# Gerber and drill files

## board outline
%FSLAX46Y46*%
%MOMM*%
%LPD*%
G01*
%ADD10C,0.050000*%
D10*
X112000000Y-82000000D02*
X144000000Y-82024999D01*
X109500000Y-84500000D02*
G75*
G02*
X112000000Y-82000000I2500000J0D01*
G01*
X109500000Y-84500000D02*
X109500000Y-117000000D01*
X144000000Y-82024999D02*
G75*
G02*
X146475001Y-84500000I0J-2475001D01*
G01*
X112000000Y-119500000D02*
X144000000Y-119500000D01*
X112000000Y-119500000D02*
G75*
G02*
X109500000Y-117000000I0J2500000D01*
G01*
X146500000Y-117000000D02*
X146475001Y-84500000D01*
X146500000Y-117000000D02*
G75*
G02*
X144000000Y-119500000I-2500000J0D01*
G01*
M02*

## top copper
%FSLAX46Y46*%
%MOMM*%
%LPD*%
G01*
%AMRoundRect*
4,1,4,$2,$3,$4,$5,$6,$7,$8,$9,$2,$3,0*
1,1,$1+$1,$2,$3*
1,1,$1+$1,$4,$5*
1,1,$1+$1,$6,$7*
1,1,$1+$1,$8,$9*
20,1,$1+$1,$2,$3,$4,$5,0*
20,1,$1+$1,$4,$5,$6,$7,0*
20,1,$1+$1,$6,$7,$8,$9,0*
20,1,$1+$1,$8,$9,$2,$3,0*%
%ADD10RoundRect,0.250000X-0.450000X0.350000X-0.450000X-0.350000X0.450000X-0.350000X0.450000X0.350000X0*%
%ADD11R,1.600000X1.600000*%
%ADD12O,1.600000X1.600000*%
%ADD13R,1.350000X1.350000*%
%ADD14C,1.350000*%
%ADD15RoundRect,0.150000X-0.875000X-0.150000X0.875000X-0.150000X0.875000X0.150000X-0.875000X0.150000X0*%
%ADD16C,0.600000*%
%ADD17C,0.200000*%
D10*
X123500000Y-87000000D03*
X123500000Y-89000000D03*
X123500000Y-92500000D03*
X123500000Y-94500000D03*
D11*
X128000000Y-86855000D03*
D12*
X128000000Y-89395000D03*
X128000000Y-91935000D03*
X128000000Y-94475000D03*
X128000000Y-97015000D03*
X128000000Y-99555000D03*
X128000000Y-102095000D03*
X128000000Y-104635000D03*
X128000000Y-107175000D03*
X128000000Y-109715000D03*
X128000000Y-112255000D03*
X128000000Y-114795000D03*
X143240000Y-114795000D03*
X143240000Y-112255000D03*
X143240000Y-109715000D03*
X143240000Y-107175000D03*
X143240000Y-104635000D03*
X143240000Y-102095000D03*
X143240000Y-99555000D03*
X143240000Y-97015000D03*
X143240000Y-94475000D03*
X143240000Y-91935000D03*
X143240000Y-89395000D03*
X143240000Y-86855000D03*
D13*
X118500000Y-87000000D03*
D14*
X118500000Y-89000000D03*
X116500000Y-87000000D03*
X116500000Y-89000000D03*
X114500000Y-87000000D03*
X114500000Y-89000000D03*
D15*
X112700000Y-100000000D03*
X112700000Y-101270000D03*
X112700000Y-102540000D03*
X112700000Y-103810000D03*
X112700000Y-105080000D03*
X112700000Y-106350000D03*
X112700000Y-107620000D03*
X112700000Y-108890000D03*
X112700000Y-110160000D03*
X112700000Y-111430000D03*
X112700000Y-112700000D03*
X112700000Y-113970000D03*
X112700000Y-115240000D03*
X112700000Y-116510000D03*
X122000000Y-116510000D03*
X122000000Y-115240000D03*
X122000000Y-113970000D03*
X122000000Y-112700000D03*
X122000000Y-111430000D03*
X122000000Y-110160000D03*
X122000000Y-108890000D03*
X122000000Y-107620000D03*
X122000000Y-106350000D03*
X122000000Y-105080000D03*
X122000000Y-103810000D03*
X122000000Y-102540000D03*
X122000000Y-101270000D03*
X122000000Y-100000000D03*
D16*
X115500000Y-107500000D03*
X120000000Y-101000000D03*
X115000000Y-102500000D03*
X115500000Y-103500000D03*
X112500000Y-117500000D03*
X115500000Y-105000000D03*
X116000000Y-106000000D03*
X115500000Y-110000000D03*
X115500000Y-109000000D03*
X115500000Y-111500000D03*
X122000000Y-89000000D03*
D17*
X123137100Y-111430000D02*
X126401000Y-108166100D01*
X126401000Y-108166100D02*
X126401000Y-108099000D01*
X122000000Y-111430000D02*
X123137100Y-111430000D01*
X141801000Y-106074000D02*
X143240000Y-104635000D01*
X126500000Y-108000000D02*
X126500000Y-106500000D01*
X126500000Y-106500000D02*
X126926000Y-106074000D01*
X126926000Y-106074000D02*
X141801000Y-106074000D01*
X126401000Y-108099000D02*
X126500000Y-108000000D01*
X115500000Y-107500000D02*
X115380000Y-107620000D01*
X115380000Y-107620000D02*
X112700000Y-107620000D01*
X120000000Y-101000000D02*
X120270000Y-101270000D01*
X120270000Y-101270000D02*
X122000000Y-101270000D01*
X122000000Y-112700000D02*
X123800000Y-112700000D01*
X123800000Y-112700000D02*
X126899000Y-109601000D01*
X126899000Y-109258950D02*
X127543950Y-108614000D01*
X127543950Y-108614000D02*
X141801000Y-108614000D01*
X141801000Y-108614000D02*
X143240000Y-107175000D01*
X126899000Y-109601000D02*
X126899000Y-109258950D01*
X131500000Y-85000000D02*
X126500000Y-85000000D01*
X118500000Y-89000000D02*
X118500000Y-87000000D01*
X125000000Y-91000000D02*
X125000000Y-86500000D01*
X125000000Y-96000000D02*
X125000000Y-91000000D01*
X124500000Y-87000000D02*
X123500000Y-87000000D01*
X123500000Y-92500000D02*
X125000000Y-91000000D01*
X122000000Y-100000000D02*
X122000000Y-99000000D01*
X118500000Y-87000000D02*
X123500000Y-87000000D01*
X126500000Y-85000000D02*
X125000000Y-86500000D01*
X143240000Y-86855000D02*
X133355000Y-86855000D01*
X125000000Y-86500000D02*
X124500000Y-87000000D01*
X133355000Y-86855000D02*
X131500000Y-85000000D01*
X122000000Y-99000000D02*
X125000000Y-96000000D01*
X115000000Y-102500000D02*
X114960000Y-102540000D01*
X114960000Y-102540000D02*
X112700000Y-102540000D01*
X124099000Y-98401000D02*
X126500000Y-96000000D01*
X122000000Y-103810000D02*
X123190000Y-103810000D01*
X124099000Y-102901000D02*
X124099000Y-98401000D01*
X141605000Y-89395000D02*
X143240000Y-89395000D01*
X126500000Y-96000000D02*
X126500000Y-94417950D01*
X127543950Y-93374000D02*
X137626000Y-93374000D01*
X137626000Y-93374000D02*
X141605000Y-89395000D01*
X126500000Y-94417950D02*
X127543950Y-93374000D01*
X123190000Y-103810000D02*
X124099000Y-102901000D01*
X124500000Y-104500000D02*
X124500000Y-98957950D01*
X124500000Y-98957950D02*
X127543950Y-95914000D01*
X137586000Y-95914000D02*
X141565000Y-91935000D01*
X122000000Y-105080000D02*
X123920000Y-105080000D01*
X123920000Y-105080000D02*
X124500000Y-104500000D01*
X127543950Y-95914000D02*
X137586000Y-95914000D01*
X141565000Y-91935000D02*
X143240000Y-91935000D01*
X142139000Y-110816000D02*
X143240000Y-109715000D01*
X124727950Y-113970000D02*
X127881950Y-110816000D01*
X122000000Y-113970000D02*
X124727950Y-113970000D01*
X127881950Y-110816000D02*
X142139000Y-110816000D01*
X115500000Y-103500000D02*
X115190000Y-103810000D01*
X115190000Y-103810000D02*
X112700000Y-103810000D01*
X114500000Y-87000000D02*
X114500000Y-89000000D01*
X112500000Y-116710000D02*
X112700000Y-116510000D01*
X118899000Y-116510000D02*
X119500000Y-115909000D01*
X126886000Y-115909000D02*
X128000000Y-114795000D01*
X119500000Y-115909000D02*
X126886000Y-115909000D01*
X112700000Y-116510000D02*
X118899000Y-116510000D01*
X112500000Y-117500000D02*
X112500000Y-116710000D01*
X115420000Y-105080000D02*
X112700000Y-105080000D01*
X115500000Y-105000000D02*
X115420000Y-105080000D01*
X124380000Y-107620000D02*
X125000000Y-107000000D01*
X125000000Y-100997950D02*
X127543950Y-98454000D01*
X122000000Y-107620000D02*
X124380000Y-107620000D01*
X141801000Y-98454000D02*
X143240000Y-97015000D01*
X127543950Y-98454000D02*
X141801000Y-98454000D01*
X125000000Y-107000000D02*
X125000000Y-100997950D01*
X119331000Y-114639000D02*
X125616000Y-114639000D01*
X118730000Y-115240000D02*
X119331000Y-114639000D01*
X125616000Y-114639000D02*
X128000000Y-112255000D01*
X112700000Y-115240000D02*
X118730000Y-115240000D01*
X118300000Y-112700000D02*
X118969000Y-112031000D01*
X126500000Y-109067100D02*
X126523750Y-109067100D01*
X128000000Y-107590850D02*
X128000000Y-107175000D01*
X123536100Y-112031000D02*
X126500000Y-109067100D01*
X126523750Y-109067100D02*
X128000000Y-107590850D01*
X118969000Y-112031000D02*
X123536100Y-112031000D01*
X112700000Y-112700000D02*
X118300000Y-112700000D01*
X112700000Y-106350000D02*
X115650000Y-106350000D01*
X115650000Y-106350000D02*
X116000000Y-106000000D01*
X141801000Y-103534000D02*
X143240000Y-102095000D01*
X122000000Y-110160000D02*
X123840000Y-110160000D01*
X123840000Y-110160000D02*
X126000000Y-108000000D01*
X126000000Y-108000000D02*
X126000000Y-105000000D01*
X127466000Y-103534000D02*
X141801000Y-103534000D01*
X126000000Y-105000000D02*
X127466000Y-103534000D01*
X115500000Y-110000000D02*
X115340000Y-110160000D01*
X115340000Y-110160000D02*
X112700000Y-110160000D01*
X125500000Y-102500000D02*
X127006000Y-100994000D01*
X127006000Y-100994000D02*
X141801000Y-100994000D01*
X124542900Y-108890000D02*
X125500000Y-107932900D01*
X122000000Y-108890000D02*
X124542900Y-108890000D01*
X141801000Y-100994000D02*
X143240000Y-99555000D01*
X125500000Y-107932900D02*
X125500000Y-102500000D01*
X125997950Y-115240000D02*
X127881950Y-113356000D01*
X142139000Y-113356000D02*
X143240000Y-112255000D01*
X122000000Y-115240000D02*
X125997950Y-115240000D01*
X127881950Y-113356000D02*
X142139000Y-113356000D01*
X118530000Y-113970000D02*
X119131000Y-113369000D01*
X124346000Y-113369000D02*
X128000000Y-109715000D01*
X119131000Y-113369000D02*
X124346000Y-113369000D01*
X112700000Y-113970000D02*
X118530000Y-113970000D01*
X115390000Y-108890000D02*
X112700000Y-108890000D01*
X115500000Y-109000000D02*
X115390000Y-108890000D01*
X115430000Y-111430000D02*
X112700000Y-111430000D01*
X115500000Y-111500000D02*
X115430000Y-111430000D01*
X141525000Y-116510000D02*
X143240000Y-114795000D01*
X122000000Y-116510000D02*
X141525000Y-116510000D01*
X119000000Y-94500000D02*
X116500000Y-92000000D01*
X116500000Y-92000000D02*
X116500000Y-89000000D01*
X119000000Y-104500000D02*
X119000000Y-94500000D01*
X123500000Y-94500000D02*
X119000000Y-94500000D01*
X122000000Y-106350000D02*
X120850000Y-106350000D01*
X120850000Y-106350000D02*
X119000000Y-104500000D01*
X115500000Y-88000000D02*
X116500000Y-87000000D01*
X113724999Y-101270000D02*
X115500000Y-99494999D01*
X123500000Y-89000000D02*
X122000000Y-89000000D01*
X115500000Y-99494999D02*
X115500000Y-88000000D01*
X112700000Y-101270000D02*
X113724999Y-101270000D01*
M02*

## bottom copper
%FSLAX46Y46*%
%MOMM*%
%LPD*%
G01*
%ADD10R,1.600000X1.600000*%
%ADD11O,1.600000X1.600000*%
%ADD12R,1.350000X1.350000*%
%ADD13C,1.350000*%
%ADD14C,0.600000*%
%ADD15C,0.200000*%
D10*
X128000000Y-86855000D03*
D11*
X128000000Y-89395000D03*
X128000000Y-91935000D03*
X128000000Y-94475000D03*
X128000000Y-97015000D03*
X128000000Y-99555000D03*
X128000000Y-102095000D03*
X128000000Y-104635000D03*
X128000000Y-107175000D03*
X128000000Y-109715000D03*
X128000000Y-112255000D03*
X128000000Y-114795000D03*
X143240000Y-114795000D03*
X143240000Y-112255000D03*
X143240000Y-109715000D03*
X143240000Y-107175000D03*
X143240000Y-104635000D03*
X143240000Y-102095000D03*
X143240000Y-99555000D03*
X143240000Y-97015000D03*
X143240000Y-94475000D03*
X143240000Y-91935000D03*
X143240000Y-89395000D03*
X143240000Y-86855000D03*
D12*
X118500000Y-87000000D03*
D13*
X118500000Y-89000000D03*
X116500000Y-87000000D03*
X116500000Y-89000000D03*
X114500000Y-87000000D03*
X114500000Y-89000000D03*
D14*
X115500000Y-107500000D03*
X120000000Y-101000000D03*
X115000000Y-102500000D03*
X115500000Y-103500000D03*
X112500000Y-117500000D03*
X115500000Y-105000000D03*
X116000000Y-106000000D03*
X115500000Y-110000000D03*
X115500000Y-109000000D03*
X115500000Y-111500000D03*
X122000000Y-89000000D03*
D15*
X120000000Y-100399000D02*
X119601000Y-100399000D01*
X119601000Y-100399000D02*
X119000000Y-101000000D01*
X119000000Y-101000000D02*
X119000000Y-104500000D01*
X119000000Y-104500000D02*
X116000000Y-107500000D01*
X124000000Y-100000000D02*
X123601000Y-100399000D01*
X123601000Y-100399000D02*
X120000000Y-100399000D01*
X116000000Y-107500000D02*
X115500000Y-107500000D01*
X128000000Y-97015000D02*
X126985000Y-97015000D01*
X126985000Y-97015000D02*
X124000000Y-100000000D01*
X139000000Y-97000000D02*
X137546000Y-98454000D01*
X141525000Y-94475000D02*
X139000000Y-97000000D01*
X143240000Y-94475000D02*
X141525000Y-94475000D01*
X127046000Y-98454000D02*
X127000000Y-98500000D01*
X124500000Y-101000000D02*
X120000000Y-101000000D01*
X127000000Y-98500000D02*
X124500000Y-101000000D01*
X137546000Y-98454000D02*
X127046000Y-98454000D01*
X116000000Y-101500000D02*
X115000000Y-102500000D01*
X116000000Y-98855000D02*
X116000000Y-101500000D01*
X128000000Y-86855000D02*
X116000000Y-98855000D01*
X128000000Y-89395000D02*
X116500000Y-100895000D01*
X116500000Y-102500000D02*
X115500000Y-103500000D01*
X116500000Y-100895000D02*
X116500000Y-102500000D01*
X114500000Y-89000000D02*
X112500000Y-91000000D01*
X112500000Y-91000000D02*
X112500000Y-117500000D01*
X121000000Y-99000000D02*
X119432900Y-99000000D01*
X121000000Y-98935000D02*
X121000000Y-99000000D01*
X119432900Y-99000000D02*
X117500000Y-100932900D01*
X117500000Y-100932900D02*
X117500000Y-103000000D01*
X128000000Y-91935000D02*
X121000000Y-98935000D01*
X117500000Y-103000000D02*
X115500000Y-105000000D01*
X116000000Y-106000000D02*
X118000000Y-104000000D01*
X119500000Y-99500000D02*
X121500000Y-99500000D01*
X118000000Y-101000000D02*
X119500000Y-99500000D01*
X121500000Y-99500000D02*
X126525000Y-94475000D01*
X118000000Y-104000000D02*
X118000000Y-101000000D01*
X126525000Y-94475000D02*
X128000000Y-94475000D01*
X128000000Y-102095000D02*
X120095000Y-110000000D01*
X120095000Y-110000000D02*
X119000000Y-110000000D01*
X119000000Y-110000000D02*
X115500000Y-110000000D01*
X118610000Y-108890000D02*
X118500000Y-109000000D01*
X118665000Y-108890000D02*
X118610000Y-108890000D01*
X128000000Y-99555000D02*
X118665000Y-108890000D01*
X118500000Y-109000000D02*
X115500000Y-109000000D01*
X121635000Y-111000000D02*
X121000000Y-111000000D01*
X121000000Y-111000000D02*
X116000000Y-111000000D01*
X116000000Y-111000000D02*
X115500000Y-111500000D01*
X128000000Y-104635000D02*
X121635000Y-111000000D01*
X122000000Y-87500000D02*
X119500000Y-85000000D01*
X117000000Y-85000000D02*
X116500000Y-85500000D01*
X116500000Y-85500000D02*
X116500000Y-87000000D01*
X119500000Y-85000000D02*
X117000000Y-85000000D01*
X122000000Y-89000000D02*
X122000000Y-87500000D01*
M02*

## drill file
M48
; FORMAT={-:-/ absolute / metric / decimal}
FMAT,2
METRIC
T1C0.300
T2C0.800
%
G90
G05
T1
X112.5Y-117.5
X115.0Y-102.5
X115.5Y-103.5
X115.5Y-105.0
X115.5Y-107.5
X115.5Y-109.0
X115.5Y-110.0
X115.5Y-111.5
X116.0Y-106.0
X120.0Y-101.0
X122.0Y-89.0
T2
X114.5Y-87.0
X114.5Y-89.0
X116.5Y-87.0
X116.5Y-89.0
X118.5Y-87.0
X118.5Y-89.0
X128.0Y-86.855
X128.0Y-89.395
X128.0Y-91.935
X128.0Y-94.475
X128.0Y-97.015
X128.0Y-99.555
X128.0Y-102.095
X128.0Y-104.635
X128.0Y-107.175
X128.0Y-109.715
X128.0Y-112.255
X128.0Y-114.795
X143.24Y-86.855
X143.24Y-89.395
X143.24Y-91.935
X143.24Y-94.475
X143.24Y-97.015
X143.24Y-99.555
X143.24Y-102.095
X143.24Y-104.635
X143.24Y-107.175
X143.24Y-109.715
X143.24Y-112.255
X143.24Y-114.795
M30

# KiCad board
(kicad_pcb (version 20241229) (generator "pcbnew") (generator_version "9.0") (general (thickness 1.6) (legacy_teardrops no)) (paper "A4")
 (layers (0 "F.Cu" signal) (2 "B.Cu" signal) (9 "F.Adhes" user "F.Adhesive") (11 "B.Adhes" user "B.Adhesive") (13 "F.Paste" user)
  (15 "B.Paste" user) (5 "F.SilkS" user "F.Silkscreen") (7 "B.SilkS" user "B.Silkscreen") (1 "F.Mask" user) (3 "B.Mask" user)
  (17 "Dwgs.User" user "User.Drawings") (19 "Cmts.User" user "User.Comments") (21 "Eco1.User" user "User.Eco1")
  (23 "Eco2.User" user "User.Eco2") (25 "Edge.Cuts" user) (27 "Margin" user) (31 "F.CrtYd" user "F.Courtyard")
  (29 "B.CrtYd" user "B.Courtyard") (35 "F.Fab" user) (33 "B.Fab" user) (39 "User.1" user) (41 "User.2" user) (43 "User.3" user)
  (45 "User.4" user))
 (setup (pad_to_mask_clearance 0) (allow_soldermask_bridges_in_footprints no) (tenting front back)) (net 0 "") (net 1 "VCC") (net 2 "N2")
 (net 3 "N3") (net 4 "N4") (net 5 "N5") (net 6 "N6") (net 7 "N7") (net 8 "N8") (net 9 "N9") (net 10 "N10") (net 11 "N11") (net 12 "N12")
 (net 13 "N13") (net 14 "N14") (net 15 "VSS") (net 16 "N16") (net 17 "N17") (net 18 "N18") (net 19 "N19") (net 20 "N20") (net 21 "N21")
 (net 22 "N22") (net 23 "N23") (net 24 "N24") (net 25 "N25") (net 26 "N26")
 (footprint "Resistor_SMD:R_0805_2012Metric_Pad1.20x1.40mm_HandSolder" (layer "F.Cu") (at 123.5 88 -90)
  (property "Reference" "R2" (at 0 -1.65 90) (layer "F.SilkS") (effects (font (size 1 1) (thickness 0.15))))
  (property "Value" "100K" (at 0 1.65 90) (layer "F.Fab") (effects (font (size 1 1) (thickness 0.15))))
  (pad "1" smd roundrect (at -1 0 270) (size 1.2 1.4) (layers "F.Cu" "F.Mask" "F.Paste") (roundrect_rratio 0.208333) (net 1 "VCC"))
  (pad "2" smd roundrect (at 1 0 270) (size 1.2 1.4) (layers "F.Cu" "F.Mask" "F.Paste") (roundrect_rratio 0.208333) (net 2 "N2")))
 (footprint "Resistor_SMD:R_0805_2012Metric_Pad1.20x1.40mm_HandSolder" (layer "F.Cu") (at 123.5 93.5 -90)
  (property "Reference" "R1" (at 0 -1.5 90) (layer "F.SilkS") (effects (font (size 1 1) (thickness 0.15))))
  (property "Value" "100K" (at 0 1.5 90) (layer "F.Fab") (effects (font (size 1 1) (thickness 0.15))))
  (pad "1" smd roundrect (at -1 0 270) (size 1.2 1.4) (layers "F.Cu" "F.Mask" "F.Paste") (roundrect_rratio 0.208333) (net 1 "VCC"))
  (pad "2" smd roundrect (at 1 0 270) (size 1.2 1.4) (layers "F.Cu" "F.Mask" "F.Paste") (roundrect_rratio 0.208333) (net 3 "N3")))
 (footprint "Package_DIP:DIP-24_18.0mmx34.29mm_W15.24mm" (layer "F.Cu") (at 128 86.855)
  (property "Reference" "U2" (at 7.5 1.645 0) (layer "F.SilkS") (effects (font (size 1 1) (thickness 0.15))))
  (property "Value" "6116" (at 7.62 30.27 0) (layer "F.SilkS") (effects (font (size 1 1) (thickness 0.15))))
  (pad "1" thru_hole rect (at 0 0) (size 1.6 1.6) (drill 0.8) (layers "*.Cu" "*.Mask") (remove_unused_layers no) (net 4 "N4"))
  (pad "2" thru_hole oval (at 0 2.54) (size 1.6 1.6) (drill 0.8) (layers "*.Cu" "*.Mask") (remove_unused_layers no) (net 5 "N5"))
  (pad "3" thru_hole oval (at 0 5.08) (size 1.6 1.6) (drill 0.8) (layers "*.Cu" "*.Mask") (remove_unused_layers no) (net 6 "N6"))
  (pad "4" thru_hole oval (at 0 7.62) (size 1.6 1.6) (drill 0.8) (layers "*.Cu" "*.Mask") (remove_unused_layers no) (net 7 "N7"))
  (pad "5" thru_hole oval (at 0 10.16) (size 1.6 1.6) (drill 0.8) (layers "*.Cu" "*.Mask") (remove_unused_layers no) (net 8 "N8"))
  (pad "6" thru_hole oval (at 0 12.7) (size 1.6 1.6) (drill 0.8) (layers "*.Cu" "*.Mask") (remove_unused_layers no) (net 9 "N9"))
  (pad "7" thru_hole oval (at 0 15.24) (size 1.6 1.6) (drill 0.8) (layers "*.Cu" "*.Mask") (remove_unused_layers no) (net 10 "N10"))
  (pad "8" thru_hole oval (at 0 17.78) (size 1.6 1.6) (drill 0.8) (layers "*.Cu" "*.Mask") (remove_unused_layers no) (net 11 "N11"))
  (pad "9" thru_hole oval (at 0 20.32) (size 1.6 1.6) (drill 0.8) (layers "*.Cu" "*.Mask") (remove_unused_layers no) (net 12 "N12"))
  (pad "10" thru_hole oval (at 0 22.86) (size 1.6 1.6) (drill 0.8) (layers "*.Cu" "*.Mask") (remove_unused_layers no) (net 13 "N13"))
  (pad "11" thru_hole oval (at 0 25.4) (size 1.6 1.6) (drill 0.8) (layers "*.Cu" "*.Mask") (remove_unused_layers no) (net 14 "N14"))
  (pad "12" thru_hole oval (at 0 27.94) (size 1.6 1.6) (drill 0.8) (layers "*.Cu" "*.Mask") (remove_unused_layers no) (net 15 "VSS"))
  (pad "13" thru_hole oval (at 15.24 27.94) (size 1.6 1.6) (drill 0.8) (layers "*.Cu" "*.Mask") (remove_unused_layers no) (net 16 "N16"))
  (pad "14" thru_hole oval (at 15.24 25.4) (size 1.6 1.6) (drill 0.8) (layers "*.Cu" "*.Mask") (remove_unused_layers no) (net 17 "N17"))
  (pad "15" thru_hole oval (at 15.24 22.86) (size 1.6 1.6) (drill 0.8) (layers "*.Cu" "*.Mask") (remove_unused_layers no) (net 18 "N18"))
  (pad "16" thru_hole oval (at 15.24 20.32) (size 1.6 1.6) (drill 0.8) (layers "*.Cu" "*.Mask") (remove_unused_layers no) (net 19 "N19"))
  (pad "17" thru_hole oval (at 15.24 17.78) (size 1.6 1.6) (drill 0.8) (layers "*.Cu" "*.Mask") (remove_unused_layers no) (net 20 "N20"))
  (pad "18" thru_hole oval (at 15.24 15.24) (size 1.6 1.6) (drill 0.8) (layers "*.Cu" "*.Mask") (remove_unused_layers no) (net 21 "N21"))
  (pad "19" thru_hole oval (at 15.24 12.7) (size 1.6 1.6) (drill 0.8) (layers "*.Cu" "*.Mask") (remove_unused_layers no) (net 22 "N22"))
  (pad "20" thru_hole oval (at 15.24 10.16) (size 1.6 1.6) (drill 0.8) (layers "*.Cu" "*.Mask") (remove_unused_layers no) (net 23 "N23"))
  (pad "21" thru_hole oval (at 15.24 7.62) (size 1.6 1.6) (drill 0.8) (layers "*.Cu" "*.Mask") (remove_unused_layers no) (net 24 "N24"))
  (pad "22" thru_hole oval (at 15.24 5.08) (size 1.6 1.6) (drill 0.8) (layers "*.Cu" "*.Mask") (remove_unused_layers no) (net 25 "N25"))
  (pad "23" thru_hole oval (at 15.24 2.54) (size 1.6 1.6) (drill 0.8) (layers "*.Cu" "*.Mask") (remove_unused_layers no) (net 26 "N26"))
  (pad "24" thru_hole oval (at 15.24 0) (size 1.6 1.6) (drill 0.8) (layers "*.Cu" "*.Mask") (remove_unused_layers no) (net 1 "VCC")))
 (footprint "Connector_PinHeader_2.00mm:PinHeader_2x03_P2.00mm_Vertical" (layer "F.Cu") (at 118.5 87 -90)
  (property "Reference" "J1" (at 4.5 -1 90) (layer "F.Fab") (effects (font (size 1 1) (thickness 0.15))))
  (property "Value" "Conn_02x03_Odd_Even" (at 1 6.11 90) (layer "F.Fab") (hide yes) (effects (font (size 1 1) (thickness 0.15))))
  (pad "1" thru_hole rect (at 0 0 270) (size 1.35 1.35) (drill 0.8) (layers "*.Cu" "*.Mask") (remove_unused_layers no) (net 1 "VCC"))
  (pad "2" thru_hole circle (at 2 0 270) (size 1.35 1.35) (drill 0.8) (layers "*.Cu" "*.Mask") (remove_unused_layers no) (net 1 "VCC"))
  (pad "3" thru_hole circle (at 0 2 270) (size 1.35 1.35) (drill 0.8) (layers "*.Cu" "*.Mask") (remove_unused_layers no) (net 2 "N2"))
  (pad "4" thru_hole circle (at 2 2 270) (size 1.35 1.35) (drill 0.8) (layers "*.Cu" "*.Mask") (remove_unused_layers no) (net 3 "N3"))
  (pad "5" thru_hole circle (at 0 4 270) (size 1.35 1.35) (drill 0.8) (layers "*.Cu" "*.Mask") (remove_unused_layers no) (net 15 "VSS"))
  (pad "6" thru_hole circle (at 2 4 270) (size 1.35 1.35) (drill 0.8) (layers "*.Cu" "*.Mask") (remove_unused_layers no) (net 15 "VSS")))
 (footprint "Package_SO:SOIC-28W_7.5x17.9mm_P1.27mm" (layer "F.Cu") (at 117.35 108.255)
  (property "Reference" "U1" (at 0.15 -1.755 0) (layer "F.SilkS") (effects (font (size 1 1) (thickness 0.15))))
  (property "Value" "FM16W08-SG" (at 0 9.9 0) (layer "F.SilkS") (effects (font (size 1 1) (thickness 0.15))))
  (pad "1" smd roundrect (at -4.65 -8.255) (size 2.05 0.6) (layers "F.Cu" "F.Mask" "F.Paste") (roundrect_rratio 0.25))
  (pad "2" smd roundrect (at -4.65 -6.985) (size 2.05 0.6) (layers "F.Cu" "F.Mask" "F.Paste") (roundrect_rratio 0.25) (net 2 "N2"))
  (pad "3" smd roundrect (at -4.65 -5.715) (size 2.05 0.6) (layers "F.Cu" "F.Mask" "F.Paste") (roundrect_rratio 0.25) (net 4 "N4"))
  (pad "4" smd roundrect (at -4.65 -4.445) (size 2.05 0.6) (layers "F.Cu" "F.Mask" "F.Paste") (roundrect_rratio 0.25) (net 5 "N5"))
  (pad "5" smd roundrect (at -4.65 -3.175) (size 2.05 0.6) (layers "F.Cu" "F.Mask" "F.Paste") (roundrect_rratio 0.25) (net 6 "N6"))
  (pad "6" smd roundrect (at -4.65 -1.905) (size 2.05 0.6) (layers "F.Cu" "F.Mask" "F.Paste") (roundrect_rratio 0.25) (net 7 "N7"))
  (pad "7" smd roundrect (at -4.65 -0.635) (size 2.05 0.6) (layers "F.Cu" "F.Mask" "F.Paste") (roundrect_rratio 0.25) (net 8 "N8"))
  (pad "8" smd roundrect (at -4.65 0.635) (size 2.05 0.6) (layers "F.Cu" "F.Mask" "F.Paste") (roundrect_rratio 0.25) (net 9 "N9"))
  (pad "9" smd roundrect (at -4.65 1.905) (size 2.05 0.6) (layers "F.Cu" "F.Mask" "F.Paste") (roundrect_rratio 0.25) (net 10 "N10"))
  (pad "10" smd roundrect (at -4.65 3.175) (size 2.05 0.6) (layers "F.Cu" "F.Mask" "F.Paste") (roundrect_rratio 0.25) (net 11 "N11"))
  (pad "11" smd roundrect (at -4.65 4.445) (size 2.05 0.6) (layers "F.Cu" "F.Mask" "F.Paste") (roundrect_rratio 0.25) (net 12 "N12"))
  (pad "12" smd roundrect (at -4.65 5.715) (size 2.05 0.6) (layers "F.Cu" "F.Mask" "F.Paste") (roundrect_rratio 0.25) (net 13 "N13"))
  (pad "13" smd roundrect (at -4.65 6.985) (size 2.05 0.6) (layers "F.Cu" "F.Mask" "F.Paste") (roundrect_rratio 0.25) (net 14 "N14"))
  (pad "14" smd roundrect (at -4.65 8.255) (size 2.05 0.6) (layers "F.Cu" "F.Mask" "F.Paste") (roundrect_rratio 0.25) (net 15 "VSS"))
  (pad "15" smd roundrect (at 4.65 8.255) (size 2.05 0.6) (layers "F.Cu" "F.Mask" "F.Paste") (roundrect_rratio 0.25) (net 16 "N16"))
  (pad "16" smd roundrect (at 4.65 6.985) (size 2.05 0.6) (layers "F.Cu" "F.Mask" "F.Paste") (roundrect_rratio 0.25) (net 17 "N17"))
  (pad "17" smd roundrect (at 4.65 5.715) (size 2.05 0.6) (layers "F.Cu" "F.Mask" "F.Paste") (roundrect_rratio 0.25) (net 18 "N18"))
  (pad "18" smd roundrect (at 4.65 4.445) (size 2.05 0.6) (layers "F.Cu" "F.Mask" "F.Paste") (roundrect_rratio 0.25) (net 19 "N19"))
  (pad "19" smd roundrect (at 4.65 3.175) (size 2.05 0.6) (layers "F.Cu" "F.Mask" "F.Paste") (roundrect_rratio 0.25) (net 20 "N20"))
  (pad "20" smd roundrect (at 4.65 1.905) (size 2.05 0.6) (layers "F.Cu" "F.Mask" "F.Paste") (roundrect_rratio 0.25) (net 21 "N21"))
  (pad "21" smd roundrect (at 4.65 0.635) (size 2.05 0.6) (layers "F.Cu" "F.Mask" "F.Paste") (roundrect_rratio 0.25) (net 22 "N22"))
  (pad "22" smd roundrect (at 4.65 -0.635) (size 2.05 0.6) (layers "F.Cu" "F.Mask" "F.Paste") (roundrect_rratio 0.25) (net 23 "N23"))
  (pad "23" smd roundrect (at 4.65 -1.905) (size 2.05 0.6) (layers "F.Cu" "F.Mask" "F.Paste") (roundrect_rratio 0.25) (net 3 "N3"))
  (pad "24" smd roundrect (at 4.65 -3.175) (size 2.05 0.6) (layers "F.Cu" "F.Mask" "F.Paste") (roundrect_rratio 0.25) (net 25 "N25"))
  (pad "25" smd roundrect (at 4.65 -4.445) (size 2.05 0.6) (layers "F.Cu" "F.Mask" "F.Paste") (roundrect_rratio 0.25) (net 26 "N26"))
  (pad "26" smd roundrect (at 4.65 -5.715) (size 2.05 0.6) (layers "F.Cu" "F.Mask" "F.Paste") (roundrect_rratio 0.25))
  (pad "27" smd roundrect (at 4.65 -6.985) (size 2.05 0.6) (layers "F.Cu" "F.Mask" "F.Paste") (roundrect_rratio 0.25) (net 24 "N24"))
  (pad "28" smd roundrect (at 4.65 -8.255) (size 2.05 0.6) (layers "F.Cu" "F.Mask" "F.Paste") (roundrect_rratio 0.25) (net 1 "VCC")))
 (gr_line (start 112 82) (end 144 82.024999) (stroke (width 0.05) (type default)) (layer "Edge.Cuts"))
 (gr_arc (start 109.5 84.5) (mid 110.232233 82.732233) (end 112 82) (stroke (width 0.05) (type default)) (layer "Edge.Cuts"))
 (gr_line (start 109.5 84.5) (end 109.5 117) (stroke (width 0.05) (type default)) (layer "Edge.Cuts"))
 (gr_arc (start 144 82.024999) (mid 145.75009 82.74991) (end 146.475001 84.5) (stroke (width 0.05) (type solid)) (layer "Edge.Cuts"))
 (gr_line (start 112 119.5) (end 144 119.5) (stroke (width 0.05) (type default)) (layer "Edge.Cuts"))
 (gr_arc (start 112 119.5) (mid 110.232233 118.767767) (end 109.5 117) (stroke (width 0.05) (type solid)) (layer "Edge.Cuts"))
 (gr_line (start 146.5 117) (end 146.475001 84.5) (stroke (width 0.05) (type default)) (layer "Edge.Cuts"))
 (gr_arc (start 146.5 117) (mid 145.767767 118.767767) (end 144 119.5) (stroke (width 0.05) (type default)) (layer "Edge.Cuts"))
 (segment (start 123.1371 111.43) (end 126.401 108.1661) (width 0.2) (layer "F.Cu") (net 20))
 (segment (start 126.401 108.1661) (end 126.401 108.099) (width 0.2) (layer "F.Cu") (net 20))
 (segment (start 122 111.43) (end 123.1371 111.43) (width 0.2) (layer "F.Cu") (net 20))
 (segment (start 141.801 106.074) (end 143.24 104.635) (width 0.2) (layer "F.Cu") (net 20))
 (segment (start 126.5 108) (end 126.5 106.5) (width 0.2) (layer "F.Cu") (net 20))
 (segment (start 126.5 106.5) (end 126.926 106.074) (width 0.2) (layer "F.Cu") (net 20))
 (segment (start 126.926 106.074) (end 141.801 106.074) (width 0.2) (layer "F.Cu") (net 20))
 (segment (start 126.401 108.099) (end 126.5 108) (width 0.2) (layer "F.Cu") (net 20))
 (segment (start 115.5 107.5) (end 115.38 107.62) (width 0.2) (layer "F.Cu") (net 8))
 (segment (start 115.38 107.62) (end 112.7 107.62) (width 0.2) (layer "F.Cu") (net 8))
 (via (at 115.5 107.5) (size 0.6) (drill 0.3) (layers "F.Cu" "B.Cu") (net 8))
 (segment (start 120 100.399) (end 119.601 100.399) (width 0.2) (layer "B.Cu") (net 8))
 (segment (start 119.601 100.399) (end 119 101) (width 0.2) (layer "B.Cu") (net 8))
 (segment (start 119 101) (end 119 104.5) (width 0.2) (layer "B.Cu") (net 8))
 (segment (start 119 104.5) (end 116 107.5) (width 0.2) (layer "B.Cu") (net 8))
 (segment (start 124 100) (end 123.601 100.399) (width 0.2) (layer "B.Cu") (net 8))
 (segment (start 123.601 100.399) (end 120 100.399) (width 0.2) (layer "B.Cu") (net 8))
 (segment (start 116 107.5) (end 115.5 107.5) (width 0.2) (layer "B.Cu") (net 8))
 (segment (start 128 97.015) (end 126.985 97.015) (width 0.2) (layer "B.Cu") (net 8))
 (segment (start 126.985 97.015) (end 124 100) (width 0.2) (layer "B.Cu") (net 8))
 (segment (start 120 101) (end 120.27 101.27) (width 0.2) (layer "F.Cu") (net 24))
 (segment (start 120.27 101.27) (end 122 101.27) (width 0.2) (layer "F.Cu") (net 24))
 (via (at 120 101) (size 0.6) (drill 0.3) (layers "F.Cu" "B.Cu") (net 24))
 (segment (start 139 97) (end 137.546 98.454) (width 0.2) (layer "B.Cu") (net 24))
 (segment (start 141.525 94.475) (end 139 97) (width 0.2) (layer "B.Cu") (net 24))
 (segment (start 143.24 94.475) (end 141.525 94.475) (width 0.2) (layer "B.Cu") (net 24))
 (segment (start 127.046 98.454) (end 127 98.5) (width 0.2) (layer "B.Cu") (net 24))
 (segment (start 124.5 101) (end 120 101) (width 0.2) (layer "B.Cu") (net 24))
 (segment (start 127 98.5) (end 124.5 101) (width 0.2) (layer "B.Cu") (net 24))
 (segment (start 137.546 98.454) (end 127.046 98.454) (width 0.2) (layer "B.Cu") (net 24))
 (segment (start 122 112.7) (end 123.8 112.7) (width 0.2) (layer "F.Cu") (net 19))
 (segment (start 123.8 112.7) (end 126.899 109.601) (width 0.2) (layer "F.Cu") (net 19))
 (segment (start 126.899 109.25895) (end 127.54395 108.614) (width 0.2) (layer "F.Cu") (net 19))
 (segment (start 127.54395 108.614) (end 141.801 108.614) (width 0.2) (layer "F.Cu") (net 19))
 (segment (start 141.801 108.614) (end 143.24 107.175) (width 0.2) (layer "F.Cu") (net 19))
 (segment (start 126.899 109.601) (end 126.899 109.25895) (width 0.2) (layer "F.Cu") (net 19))
 (segment (start 131.5 85) (end 126.5 85) (width 0.2) (layer "F.Cu") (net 1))
 (segment (start 118.5 89) (end 118.5 87) (width 0.2) (layer "F.Cu") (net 1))
 (segment (start 125 91) (end 125 86.5) (width 0.2) (layer "F.Cu") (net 1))
 (segment (start 125 96) (end 125 91) (width 0.2) (layer "F.Cu") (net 1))
 (segment (start 124.5 87) (end 123.5 87) (width 0.2) (layer "F.Cu") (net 1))
 (segment (start 123.5 92.5) (end 125 91) (width 0.2) (layer "F.Cu") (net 1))
 (segment (start 122 100) (end 122 99) (width 0.2) (layer "F.Cu") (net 1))
 (segment (start 118.5 87) (end 123.5 87) (width 0.2) (layer "F.Cu") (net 1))
 (segment (start 126.5 85) (end 125 86.5) (width 0.2) (layer "F.Cu") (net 1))
 (segment (start 143.24 86.855) (end 133.355 86.855) (width 0.2) (layer "F.Cu") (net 1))
 (segment (start 125 86.5) (end 124.5 87) (width 0.2) (layer "F.Cu") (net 1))
 (segment (start 133.355 86.855) (end 131.5 85) (width 0.2) (layer "F.Cu") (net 1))
 (segment (start 122 99) (end 125 96) (width 0.2) (layer "F.Cu") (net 1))
 (segment (start 115 102.5) (end 114.96 102.54) (width 0.2) (layer "F.Cu") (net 4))
 (segment (start 114.96 102.54) (end 112.7 102.54) (width 0.2) (layer "F.Cu") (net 4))
 (via (at 115 102.5) (size 0.6) (drill 0.3) (layers "F.Cu" "B.Cu") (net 4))
 (segment (start 116 101.5) (end 115 102.5) (width 0.2) (layer "B.Cu") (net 4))
 (segment (start 116 98.855) (end 116 101.5) (width 0.2) (layer "B.Cu") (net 4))
 (segment (start 128 86.855) (end 116 98.855) (width 0.2) (layer "B.Cu") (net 4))
 (segment (start 124.099 98.401) (end 126.5 96) (width 0.2) (layer "F.Cu") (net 26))
 (segment (start 122 103.81) (end 123.19 103.81) (width 0.2) (layer "F.Cu") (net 26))
 (segment (start 124.099 102.901) (end 124.099 98.401) (width 0.2) (layer "F.Cu") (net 26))
 (segment (start 141.605 89.395) (end 143.24 89.395) (width 0.2) (layer "F.Cu") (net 26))
 (segment (start 126.5 96) (end 126.5 94.41795) (width 0.2) (layer "F.Cu") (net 26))
 (segment (start 127.54395 93.374) (end 137.626 93.374) (width 0.2) (layer "F.Cu") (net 26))
 (segment (start 137.626 93.374) (end 141.605 89.395) (width 0.2) (layer "F.Cu") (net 26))
 (segment (start 126.5 94.41795) (end 127.54395 93.374) (width 0.2) (layer "F.Cu") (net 26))
 (segment (start 123.19 103.81) (end 124.099 102.901) (width 0.2) (layer "F.Cu") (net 26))
 (segment (start 124.5 104.5) (end 124.5 98.95795) (width 0.2) (layer "F.Cu") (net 25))
 (segment (start 124.5 98.95795) (end 127.54395 95.914) (width 0.2) (layer "F.Cu") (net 25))
 (segment (start 137.586 95.914) (end 141.565 91.935) (width 0.2) (layer "F.Cu") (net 25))
 (segment (start 122 105.08) (end 123.92 105.08) (width 0.2) (layer "F.Cu") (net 25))
 (segment (start 123.92 105.08) (end 124.5 104.5) (width 0.2) (layer "F.Cu") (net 25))
 (segment (start 127.54395 95.914) (end 137.586 95.914) (width 0.2) (layer "F.Cu") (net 25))
 (segment (start 141.565 91.935) (end 143.24 91.935) (width 0.2) (layer "F.Cu") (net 25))
 (segment (start 142.139 110.816) (end 143.24 109.715) (width 0.2) (layer "F.Cu") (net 18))
 (segment (start 124.72795 113.97) (end 127.88195 110.816) (width 0.2) (layer "F.Cu") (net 18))
 (segment (start 122 113.97) (end 124.72795 113.97) (width 0.2) (layer "F.Cu") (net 18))
 (segment (start 127.88195 110.816) (end 142.139 110.816) (width 0.2) (layer "F.Cu") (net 18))
 (segment (start 115.5 103.5) (end 115.19 103.81) (width 0.2) (layer "F.Cu") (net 5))
 (segment (start 115.19 103.81) (end 112.7 103.81) (width 0.2) (layer "F.Cu") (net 5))
 (via (at 115.5 103.5) (size 0.6) (drill 0.3) (layers "F.Cu" "B.Cu") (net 5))
 (segment (start 128 89.395) (end 116.5 100.895) (width 0.2) (layer "B.Cu") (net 5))
 (segment (start 116.5 102.5) (end 115.5 103.5) (width 0.2) (layer "B.Cu") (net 5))
 (segment (start 116.5 100.895) (end 116.5 102.5) (width 0.2) (layer "B.Cu") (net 5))
 (segment (start 114.5 87) (end 114.5 89) (width 0.2) (layer "F.Cu") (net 15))
 (segment (start 112.5 116.71) (end 112.7 116.51) (width 0.2) (layer "F.Cu") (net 15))
 (segment (start 118.899 116.51) (end 119.5 115.909) (width 0.2) (layer "F.Cu") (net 15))
 (segment (start 126.886 115.909) (end 128 114.795) (width 0.2) (layer "F.Cu") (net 15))
 (segment (start 119.5 115.909) (end 126.886 115.909) (width 0.2) (layer "F.Cu") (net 15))
 (segment (start 112.7 116.51) (end 118.899 116.51) (width 0.2) (layer "F.Cu") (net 15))
 (segment (start 112.5 117.5) (end 112.5 116.71) (width 0.2) (layer "F.Cu") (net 15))
 (via (at 112.5 117.5) (size 0.6) (drill 0.3) (layers "F.Cu" "B.Cu") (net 15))
 (segment (start 114.5 89) (end 112.5 91) (width 0.2) (layer "B.Cu") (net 15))
 (segment (start 112.5 91) (end 112.5 117.5) (width 0.2) (layer "B.Cu") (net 15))
 (segment (start 115.42 105.08) (end 112.7 105.08) (width 0.2) (layer "F.Cu") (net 6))
 (segment (start 115.5 105) (end 115.42 105.08) (width 0.2) (layer "F.Cu") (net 6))
 (via (at 115.5 105) (size 0.6) (drill 0.3) (layers "F.Cu" "B.Cu") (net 6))
 (segment (start 121 99) (end 119.4329 99) (width 0.2) (layer "B.Cu") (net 6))
 (segment (start 121 98.935) (end 121 99) (width 0.2) (layer "B.Cu") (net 6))
 (segment (start 119.4329 99) (end 117.5 100.9329) (width 0.2) (layer "B.Cu") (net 6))
 (segment (start 117.5 100.9329) (end 117.5 103) (width 0.2) (layer "B.Cu") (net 6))
 (segment (start 128 91.935) (end 121 98.935) (width 0.2) (layer "B.Cu") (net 6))
 (segment (start 117.5 103) (end 115.5 105) (width 0.2) (layer "B.Cu") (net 6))
 (segment (start 124.38 107.62) (end 125 107) (width 0.2) (layer "F.Cu") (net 23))
 (segment (start 125 100.99795) (end 127.54395 98.454) (width 0.2) (layer "F.Cu") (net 23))
 (segment (start 122 107.62) (end 124.38 107.62) (width 0.2) (layer "F.Cu") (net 23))
 (segment (start 141.801 98.454) (end 143.24 97.015) (width 0.2) (layer "F.Cu") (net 23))
 (segment (start 127.54395 98.454) (end 141.801 98.454) (width 0.2) (layer "F.Cu") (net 23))
 (segment (start 125 107) (end 125 100.99795) (width 0.2) (layer "F.Cu") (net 23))
 (segment (start 119.331 114.639) (end 125.616 114.639) (width 0.2) (layer "F.Cu") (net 14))
 (segment (start 118.73 115.24) (end 119.331 114.639) (width 0.2) (layer "F.Cu") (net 14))
 (segment (start 125.616 114.639) (end 128 112.255) (width 0.2) (layer "F.Cu") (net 14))
 (segment (start 112.7 115.24) (end 118.73 115.24) (width 0.2) (layer "F.Cu") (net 14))
 (segment (start 118.3 112.7) (end 118.969 112.031) (width 0.2) (layer "F.Cu") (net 12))
 (segment (start 126.5 109.0671) (end 126.52375 109.0671) (width 0.2) (layer "F.Cu") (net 12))
 (segment (start 128 107.59085) (end 128 107.175) (width 0.2) (layer "F.Cu") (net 12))
 (segment (start 123.5361 112.031) (end 126.5 109.0671) (width 0.2) (layer "F.Cu") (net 12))
 (segment (start 126.52375 109.0671) (end 128 107.59085) (width 0.2) (layer "F.Cu") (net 12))
 (segment (start 118.969 112.031) (end 123.5361 112.031) (width 0.2) (layer "F.Cu") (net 12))
 (segment (start 112.7 112.7) (end 118.3 112.7) (width 0.2) (layer "F.Cu") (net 12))
 (segment (start 112.7 106.35) (end 115.65 106.35) (width 0.2) (layer "F.Cu") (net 7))
 (segment (start 115.65 106.35) (end 116 106) (width 0.2) (layer "F.Cu") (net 7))
 (via (at 116 106) (size 0.6) (drill 0.3) (layers "F.Cu" "B.Cu") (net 7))
 (segment (start 116 106) (end 118 104) (width 0.2) (layer "B.Cu") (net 7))
 (segment (start 119.5 99.5) (end 121.5 99.5) (width 0.2) (layer "B.Cu") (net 7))
 (segment (start 118 101) (end 119.5 99.5) (width 0.2) (layer "B.Cu") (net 7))
 (segment (start 121.5 99.5) (end 126.525 94.475) (width 0.2) (layer "B.Cu") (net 7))
 (segment (start 118 104) (end 118 101) (width 0.2) (layer "B.Cu") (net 7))
 (segment (start 126.525 94.475) (end 128 94.475) (width 0.2) (layer "B.Cu") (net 7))
 (segment (start 141.801 103.534) (end 143.24 102.095) (width 0.2) (layer "F.Cu") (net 21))
 (segment (start 122 110.16) (end 123.84 110.16) (width 0.2) (layer "F.Cu") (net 21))
 (segment (start 123.84 110.16) (end 126 108) (width 0.2) (layer "F.Cu") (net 21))
 (segment (start 126 108) (end 126 105) (width 0.2) (layer "F.Cu") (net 21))
 (segment (start 127.466 103.534) (end 141.801 103.534) (width 0.2) (layer "F.Cu") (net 21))
 (segment (start 126 105) (end 127.466 103.534) (width 0.2) (layer "F.Cu") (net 21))
 (segment (start 115.5 110) (end 115.34 110.16) (width 0.2) (layer "F.Cu") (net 10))
 (segment (start 115.34 110.16) (end 112.7 110.16) (width 0.2) (layer "F.Cu") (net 10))
 (via (at 115.5 110) (size 0.6) (drill 0.3) (layers "F.Cu" "B.Cu") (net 10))
 (segment (start 128 102.095) (end 120.095 110) (width 0.2) (layer "B.Cu") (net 10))
 (segment (start 120.095 110) (end 119 110) (width 0.2) (layer "B.Cu") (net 10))
 (segment (start 119 110) (end 115.5 110) (width 0.2) (layer "B.Cu") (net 10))
 (segment (start 125.5 102.5) (end 127.006 100.994) (width 0.2) (layer "F.Cu") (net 22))
 (segment (start 127.006 100.994) (end 141.801 100.994) (width 0.2) (layer "F.Cu") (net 22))
 (segment (start 124.5429 108.89) (end 125.5 107.9329) (width 0.2) (layer "F.Cu") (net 22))
 (segment (start 122 108.89) (end 124.5429 108.89) (width 0.2) (layer "F.Cu") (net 22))
 (segment (start 141.801 100.994) (end 143.24 99.555) (width 0.2) (layer "F.Cu") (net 22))
 (segment (start 125.5 107.9329) (end 125.5 102.5) (width 0.2) (layer "F.Cu") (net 22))
 (segment (start 125.99795 115.24) (end 127.88195 113.356) (width 0.2) (layer "F.Cu") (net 17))
 (segment (start 142.139 113.356) (end 143.24 112.255) (width 0.2) (layer "F.Cu") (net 17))
 (segment (start 122 115.24) (end 125.99795 115.24) (width 0.2) (layer "F.Cu") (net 17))
 (segment (start 127.88195 113.356) (end 142.139 113.356) (width 0.2) (layer "F.Cu") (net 17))
 (segment (start 118.53 113.97) (end 119.131 113.369) (width 0.2) (layer "F.Cu") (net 13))
 (segment (start 124.346 113.369) (end 128 109.715) (width 0.2) (layer "F.Cu") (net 13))
 (segment (start 119.131 113.369) (end 124.346 113.369) (width 0.2) (layer "F.Cu") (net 13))
 (segment (start 112.7 113.97) (end 118.53 113.97) (width 0.2) (layer "F.Cu") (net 13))
 (segment (start 115.39 108.89) (end 112.7 108.89) (width 0.2) (layer "F.Cu") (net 9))
 (segment (start 115.5 109) (end 115.39 108.89) (width 0.2) (layer "F.Cu") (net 9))
 (via (at 115.5 109) (size 0.6) (drill 0.3) (layers "F.Cu" "B.Cu") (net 9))
 (segment (start 118.61 108.89) (end 118.5 109) (width 0.2) (layer "B.Cu") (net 9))
 (segment (start 118.665 108.89) (end 118.61 108.89) (width 0.2) (layer "B.Cu") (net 9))
 (segment (start 128 99.555) (end 118.665 108.89) (width 0.2) (layer "B.Cu") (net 9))
 (segment (start 118.5 109) (end 115.5 109) (width 0.2) (layer "B.Cu") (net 9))
 (segment (start 115.43 111.43) (end 112.7 111.43) (width 0.2) (layer "F.Cu") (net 11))
 (segment (start 115.5 111.5) (end 115.43 111.43) (width 0.2) (layer "F.Cu") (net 11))
 (via (at 115.5 111.5) (size 0.6) (drill 0.3) (layers "F.Cu" "B.Cu") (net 11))
 (segment (start 121.635 111) (end 121 111) (width 0.2) (layer "B.Cu") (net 11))
 (segment (start 121 111) (end 116 111) (width 0.2) (layer "B.Cu") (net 11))
 (segment (start 116 111) (end 115.5 111.5) (width 0.2) (layer "B.Cu") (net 11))
 (segment (start 128 104.635) (end 121.635 111) (width 0.2) (layer "B.Cu") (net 11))
 (segment (start 141.525 116.51) (end 143.24 114.795) (width 0.2) (layer "F.Cu") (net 16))
 (segment (start 122 116.51) (end 141.525 116.51) (width 0.2) (layer "F.Cu") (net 16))
 (segment (start 119 94.5) (end 116.5 92) (width 0.2) (layer "F.Cu") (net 3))
 (segment (start 116.5 92) (end 116.5 89) (width 0.2) (layer "F.Cu") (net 3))
 (segment (start 119 104.5) (end 119 94.5) (width 0.2) (layer "F.Cu") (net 3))
 (segment (start 123.5 94.5) (end 119 94.5) (width 0.2) (layer "F.Cu") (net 3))
 (segment (start 122 106.35) (end 120.85 106.35) (width 0.2) (layer "F.Cu") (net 3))
 (segment (start 120.85 106.35) (end 119 104.5) (width 0.2) (layer "F.Cu") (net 3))
 (segment (start 115.5 88) (end 116.5 87) (width 0.2) (layer "F.Cu") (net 2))
 (segment (start 113.724999 101.27) (end 115.5 99.494999) (width 0.2) (layer "F.Cu") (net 2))
 (segment (start 123.5 89) (end 122 89) (width 0.2) (layer "F.Cu") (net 2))
 (segment (start 115.5 99.494999) (end 115.5 88) (width 0.2) (layer "F.Cu") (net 2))
 (segment (start 112.7 101.27) (end 113.724999 101.27) (width 0.2) (layer "F.Cu") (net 2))
 (via (at 122 89) (size 0.6) (drill 0.3) (layers "F.Cu" "B.Cu") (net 2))
 (segment (start 122 87.5) (end 119.5 85) (width 0.2) (layer "B.Cu") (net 2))
 (segment (start 117 85) (end 116.5 85.5) (width 0.2) (layer "B.Cu") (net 2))
 (segment (start 116.5 85.5) (end 116.5 87) (width 0.2) (layer "B.Cu") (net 2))
 (segment (start 119.5 85) (end 117 85) (width 0.2) (layer "B.Cu") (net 2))
 (segment (start 122 89) (end 122 87.5) (width 0.2) (layer "B.Cu") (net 2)))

